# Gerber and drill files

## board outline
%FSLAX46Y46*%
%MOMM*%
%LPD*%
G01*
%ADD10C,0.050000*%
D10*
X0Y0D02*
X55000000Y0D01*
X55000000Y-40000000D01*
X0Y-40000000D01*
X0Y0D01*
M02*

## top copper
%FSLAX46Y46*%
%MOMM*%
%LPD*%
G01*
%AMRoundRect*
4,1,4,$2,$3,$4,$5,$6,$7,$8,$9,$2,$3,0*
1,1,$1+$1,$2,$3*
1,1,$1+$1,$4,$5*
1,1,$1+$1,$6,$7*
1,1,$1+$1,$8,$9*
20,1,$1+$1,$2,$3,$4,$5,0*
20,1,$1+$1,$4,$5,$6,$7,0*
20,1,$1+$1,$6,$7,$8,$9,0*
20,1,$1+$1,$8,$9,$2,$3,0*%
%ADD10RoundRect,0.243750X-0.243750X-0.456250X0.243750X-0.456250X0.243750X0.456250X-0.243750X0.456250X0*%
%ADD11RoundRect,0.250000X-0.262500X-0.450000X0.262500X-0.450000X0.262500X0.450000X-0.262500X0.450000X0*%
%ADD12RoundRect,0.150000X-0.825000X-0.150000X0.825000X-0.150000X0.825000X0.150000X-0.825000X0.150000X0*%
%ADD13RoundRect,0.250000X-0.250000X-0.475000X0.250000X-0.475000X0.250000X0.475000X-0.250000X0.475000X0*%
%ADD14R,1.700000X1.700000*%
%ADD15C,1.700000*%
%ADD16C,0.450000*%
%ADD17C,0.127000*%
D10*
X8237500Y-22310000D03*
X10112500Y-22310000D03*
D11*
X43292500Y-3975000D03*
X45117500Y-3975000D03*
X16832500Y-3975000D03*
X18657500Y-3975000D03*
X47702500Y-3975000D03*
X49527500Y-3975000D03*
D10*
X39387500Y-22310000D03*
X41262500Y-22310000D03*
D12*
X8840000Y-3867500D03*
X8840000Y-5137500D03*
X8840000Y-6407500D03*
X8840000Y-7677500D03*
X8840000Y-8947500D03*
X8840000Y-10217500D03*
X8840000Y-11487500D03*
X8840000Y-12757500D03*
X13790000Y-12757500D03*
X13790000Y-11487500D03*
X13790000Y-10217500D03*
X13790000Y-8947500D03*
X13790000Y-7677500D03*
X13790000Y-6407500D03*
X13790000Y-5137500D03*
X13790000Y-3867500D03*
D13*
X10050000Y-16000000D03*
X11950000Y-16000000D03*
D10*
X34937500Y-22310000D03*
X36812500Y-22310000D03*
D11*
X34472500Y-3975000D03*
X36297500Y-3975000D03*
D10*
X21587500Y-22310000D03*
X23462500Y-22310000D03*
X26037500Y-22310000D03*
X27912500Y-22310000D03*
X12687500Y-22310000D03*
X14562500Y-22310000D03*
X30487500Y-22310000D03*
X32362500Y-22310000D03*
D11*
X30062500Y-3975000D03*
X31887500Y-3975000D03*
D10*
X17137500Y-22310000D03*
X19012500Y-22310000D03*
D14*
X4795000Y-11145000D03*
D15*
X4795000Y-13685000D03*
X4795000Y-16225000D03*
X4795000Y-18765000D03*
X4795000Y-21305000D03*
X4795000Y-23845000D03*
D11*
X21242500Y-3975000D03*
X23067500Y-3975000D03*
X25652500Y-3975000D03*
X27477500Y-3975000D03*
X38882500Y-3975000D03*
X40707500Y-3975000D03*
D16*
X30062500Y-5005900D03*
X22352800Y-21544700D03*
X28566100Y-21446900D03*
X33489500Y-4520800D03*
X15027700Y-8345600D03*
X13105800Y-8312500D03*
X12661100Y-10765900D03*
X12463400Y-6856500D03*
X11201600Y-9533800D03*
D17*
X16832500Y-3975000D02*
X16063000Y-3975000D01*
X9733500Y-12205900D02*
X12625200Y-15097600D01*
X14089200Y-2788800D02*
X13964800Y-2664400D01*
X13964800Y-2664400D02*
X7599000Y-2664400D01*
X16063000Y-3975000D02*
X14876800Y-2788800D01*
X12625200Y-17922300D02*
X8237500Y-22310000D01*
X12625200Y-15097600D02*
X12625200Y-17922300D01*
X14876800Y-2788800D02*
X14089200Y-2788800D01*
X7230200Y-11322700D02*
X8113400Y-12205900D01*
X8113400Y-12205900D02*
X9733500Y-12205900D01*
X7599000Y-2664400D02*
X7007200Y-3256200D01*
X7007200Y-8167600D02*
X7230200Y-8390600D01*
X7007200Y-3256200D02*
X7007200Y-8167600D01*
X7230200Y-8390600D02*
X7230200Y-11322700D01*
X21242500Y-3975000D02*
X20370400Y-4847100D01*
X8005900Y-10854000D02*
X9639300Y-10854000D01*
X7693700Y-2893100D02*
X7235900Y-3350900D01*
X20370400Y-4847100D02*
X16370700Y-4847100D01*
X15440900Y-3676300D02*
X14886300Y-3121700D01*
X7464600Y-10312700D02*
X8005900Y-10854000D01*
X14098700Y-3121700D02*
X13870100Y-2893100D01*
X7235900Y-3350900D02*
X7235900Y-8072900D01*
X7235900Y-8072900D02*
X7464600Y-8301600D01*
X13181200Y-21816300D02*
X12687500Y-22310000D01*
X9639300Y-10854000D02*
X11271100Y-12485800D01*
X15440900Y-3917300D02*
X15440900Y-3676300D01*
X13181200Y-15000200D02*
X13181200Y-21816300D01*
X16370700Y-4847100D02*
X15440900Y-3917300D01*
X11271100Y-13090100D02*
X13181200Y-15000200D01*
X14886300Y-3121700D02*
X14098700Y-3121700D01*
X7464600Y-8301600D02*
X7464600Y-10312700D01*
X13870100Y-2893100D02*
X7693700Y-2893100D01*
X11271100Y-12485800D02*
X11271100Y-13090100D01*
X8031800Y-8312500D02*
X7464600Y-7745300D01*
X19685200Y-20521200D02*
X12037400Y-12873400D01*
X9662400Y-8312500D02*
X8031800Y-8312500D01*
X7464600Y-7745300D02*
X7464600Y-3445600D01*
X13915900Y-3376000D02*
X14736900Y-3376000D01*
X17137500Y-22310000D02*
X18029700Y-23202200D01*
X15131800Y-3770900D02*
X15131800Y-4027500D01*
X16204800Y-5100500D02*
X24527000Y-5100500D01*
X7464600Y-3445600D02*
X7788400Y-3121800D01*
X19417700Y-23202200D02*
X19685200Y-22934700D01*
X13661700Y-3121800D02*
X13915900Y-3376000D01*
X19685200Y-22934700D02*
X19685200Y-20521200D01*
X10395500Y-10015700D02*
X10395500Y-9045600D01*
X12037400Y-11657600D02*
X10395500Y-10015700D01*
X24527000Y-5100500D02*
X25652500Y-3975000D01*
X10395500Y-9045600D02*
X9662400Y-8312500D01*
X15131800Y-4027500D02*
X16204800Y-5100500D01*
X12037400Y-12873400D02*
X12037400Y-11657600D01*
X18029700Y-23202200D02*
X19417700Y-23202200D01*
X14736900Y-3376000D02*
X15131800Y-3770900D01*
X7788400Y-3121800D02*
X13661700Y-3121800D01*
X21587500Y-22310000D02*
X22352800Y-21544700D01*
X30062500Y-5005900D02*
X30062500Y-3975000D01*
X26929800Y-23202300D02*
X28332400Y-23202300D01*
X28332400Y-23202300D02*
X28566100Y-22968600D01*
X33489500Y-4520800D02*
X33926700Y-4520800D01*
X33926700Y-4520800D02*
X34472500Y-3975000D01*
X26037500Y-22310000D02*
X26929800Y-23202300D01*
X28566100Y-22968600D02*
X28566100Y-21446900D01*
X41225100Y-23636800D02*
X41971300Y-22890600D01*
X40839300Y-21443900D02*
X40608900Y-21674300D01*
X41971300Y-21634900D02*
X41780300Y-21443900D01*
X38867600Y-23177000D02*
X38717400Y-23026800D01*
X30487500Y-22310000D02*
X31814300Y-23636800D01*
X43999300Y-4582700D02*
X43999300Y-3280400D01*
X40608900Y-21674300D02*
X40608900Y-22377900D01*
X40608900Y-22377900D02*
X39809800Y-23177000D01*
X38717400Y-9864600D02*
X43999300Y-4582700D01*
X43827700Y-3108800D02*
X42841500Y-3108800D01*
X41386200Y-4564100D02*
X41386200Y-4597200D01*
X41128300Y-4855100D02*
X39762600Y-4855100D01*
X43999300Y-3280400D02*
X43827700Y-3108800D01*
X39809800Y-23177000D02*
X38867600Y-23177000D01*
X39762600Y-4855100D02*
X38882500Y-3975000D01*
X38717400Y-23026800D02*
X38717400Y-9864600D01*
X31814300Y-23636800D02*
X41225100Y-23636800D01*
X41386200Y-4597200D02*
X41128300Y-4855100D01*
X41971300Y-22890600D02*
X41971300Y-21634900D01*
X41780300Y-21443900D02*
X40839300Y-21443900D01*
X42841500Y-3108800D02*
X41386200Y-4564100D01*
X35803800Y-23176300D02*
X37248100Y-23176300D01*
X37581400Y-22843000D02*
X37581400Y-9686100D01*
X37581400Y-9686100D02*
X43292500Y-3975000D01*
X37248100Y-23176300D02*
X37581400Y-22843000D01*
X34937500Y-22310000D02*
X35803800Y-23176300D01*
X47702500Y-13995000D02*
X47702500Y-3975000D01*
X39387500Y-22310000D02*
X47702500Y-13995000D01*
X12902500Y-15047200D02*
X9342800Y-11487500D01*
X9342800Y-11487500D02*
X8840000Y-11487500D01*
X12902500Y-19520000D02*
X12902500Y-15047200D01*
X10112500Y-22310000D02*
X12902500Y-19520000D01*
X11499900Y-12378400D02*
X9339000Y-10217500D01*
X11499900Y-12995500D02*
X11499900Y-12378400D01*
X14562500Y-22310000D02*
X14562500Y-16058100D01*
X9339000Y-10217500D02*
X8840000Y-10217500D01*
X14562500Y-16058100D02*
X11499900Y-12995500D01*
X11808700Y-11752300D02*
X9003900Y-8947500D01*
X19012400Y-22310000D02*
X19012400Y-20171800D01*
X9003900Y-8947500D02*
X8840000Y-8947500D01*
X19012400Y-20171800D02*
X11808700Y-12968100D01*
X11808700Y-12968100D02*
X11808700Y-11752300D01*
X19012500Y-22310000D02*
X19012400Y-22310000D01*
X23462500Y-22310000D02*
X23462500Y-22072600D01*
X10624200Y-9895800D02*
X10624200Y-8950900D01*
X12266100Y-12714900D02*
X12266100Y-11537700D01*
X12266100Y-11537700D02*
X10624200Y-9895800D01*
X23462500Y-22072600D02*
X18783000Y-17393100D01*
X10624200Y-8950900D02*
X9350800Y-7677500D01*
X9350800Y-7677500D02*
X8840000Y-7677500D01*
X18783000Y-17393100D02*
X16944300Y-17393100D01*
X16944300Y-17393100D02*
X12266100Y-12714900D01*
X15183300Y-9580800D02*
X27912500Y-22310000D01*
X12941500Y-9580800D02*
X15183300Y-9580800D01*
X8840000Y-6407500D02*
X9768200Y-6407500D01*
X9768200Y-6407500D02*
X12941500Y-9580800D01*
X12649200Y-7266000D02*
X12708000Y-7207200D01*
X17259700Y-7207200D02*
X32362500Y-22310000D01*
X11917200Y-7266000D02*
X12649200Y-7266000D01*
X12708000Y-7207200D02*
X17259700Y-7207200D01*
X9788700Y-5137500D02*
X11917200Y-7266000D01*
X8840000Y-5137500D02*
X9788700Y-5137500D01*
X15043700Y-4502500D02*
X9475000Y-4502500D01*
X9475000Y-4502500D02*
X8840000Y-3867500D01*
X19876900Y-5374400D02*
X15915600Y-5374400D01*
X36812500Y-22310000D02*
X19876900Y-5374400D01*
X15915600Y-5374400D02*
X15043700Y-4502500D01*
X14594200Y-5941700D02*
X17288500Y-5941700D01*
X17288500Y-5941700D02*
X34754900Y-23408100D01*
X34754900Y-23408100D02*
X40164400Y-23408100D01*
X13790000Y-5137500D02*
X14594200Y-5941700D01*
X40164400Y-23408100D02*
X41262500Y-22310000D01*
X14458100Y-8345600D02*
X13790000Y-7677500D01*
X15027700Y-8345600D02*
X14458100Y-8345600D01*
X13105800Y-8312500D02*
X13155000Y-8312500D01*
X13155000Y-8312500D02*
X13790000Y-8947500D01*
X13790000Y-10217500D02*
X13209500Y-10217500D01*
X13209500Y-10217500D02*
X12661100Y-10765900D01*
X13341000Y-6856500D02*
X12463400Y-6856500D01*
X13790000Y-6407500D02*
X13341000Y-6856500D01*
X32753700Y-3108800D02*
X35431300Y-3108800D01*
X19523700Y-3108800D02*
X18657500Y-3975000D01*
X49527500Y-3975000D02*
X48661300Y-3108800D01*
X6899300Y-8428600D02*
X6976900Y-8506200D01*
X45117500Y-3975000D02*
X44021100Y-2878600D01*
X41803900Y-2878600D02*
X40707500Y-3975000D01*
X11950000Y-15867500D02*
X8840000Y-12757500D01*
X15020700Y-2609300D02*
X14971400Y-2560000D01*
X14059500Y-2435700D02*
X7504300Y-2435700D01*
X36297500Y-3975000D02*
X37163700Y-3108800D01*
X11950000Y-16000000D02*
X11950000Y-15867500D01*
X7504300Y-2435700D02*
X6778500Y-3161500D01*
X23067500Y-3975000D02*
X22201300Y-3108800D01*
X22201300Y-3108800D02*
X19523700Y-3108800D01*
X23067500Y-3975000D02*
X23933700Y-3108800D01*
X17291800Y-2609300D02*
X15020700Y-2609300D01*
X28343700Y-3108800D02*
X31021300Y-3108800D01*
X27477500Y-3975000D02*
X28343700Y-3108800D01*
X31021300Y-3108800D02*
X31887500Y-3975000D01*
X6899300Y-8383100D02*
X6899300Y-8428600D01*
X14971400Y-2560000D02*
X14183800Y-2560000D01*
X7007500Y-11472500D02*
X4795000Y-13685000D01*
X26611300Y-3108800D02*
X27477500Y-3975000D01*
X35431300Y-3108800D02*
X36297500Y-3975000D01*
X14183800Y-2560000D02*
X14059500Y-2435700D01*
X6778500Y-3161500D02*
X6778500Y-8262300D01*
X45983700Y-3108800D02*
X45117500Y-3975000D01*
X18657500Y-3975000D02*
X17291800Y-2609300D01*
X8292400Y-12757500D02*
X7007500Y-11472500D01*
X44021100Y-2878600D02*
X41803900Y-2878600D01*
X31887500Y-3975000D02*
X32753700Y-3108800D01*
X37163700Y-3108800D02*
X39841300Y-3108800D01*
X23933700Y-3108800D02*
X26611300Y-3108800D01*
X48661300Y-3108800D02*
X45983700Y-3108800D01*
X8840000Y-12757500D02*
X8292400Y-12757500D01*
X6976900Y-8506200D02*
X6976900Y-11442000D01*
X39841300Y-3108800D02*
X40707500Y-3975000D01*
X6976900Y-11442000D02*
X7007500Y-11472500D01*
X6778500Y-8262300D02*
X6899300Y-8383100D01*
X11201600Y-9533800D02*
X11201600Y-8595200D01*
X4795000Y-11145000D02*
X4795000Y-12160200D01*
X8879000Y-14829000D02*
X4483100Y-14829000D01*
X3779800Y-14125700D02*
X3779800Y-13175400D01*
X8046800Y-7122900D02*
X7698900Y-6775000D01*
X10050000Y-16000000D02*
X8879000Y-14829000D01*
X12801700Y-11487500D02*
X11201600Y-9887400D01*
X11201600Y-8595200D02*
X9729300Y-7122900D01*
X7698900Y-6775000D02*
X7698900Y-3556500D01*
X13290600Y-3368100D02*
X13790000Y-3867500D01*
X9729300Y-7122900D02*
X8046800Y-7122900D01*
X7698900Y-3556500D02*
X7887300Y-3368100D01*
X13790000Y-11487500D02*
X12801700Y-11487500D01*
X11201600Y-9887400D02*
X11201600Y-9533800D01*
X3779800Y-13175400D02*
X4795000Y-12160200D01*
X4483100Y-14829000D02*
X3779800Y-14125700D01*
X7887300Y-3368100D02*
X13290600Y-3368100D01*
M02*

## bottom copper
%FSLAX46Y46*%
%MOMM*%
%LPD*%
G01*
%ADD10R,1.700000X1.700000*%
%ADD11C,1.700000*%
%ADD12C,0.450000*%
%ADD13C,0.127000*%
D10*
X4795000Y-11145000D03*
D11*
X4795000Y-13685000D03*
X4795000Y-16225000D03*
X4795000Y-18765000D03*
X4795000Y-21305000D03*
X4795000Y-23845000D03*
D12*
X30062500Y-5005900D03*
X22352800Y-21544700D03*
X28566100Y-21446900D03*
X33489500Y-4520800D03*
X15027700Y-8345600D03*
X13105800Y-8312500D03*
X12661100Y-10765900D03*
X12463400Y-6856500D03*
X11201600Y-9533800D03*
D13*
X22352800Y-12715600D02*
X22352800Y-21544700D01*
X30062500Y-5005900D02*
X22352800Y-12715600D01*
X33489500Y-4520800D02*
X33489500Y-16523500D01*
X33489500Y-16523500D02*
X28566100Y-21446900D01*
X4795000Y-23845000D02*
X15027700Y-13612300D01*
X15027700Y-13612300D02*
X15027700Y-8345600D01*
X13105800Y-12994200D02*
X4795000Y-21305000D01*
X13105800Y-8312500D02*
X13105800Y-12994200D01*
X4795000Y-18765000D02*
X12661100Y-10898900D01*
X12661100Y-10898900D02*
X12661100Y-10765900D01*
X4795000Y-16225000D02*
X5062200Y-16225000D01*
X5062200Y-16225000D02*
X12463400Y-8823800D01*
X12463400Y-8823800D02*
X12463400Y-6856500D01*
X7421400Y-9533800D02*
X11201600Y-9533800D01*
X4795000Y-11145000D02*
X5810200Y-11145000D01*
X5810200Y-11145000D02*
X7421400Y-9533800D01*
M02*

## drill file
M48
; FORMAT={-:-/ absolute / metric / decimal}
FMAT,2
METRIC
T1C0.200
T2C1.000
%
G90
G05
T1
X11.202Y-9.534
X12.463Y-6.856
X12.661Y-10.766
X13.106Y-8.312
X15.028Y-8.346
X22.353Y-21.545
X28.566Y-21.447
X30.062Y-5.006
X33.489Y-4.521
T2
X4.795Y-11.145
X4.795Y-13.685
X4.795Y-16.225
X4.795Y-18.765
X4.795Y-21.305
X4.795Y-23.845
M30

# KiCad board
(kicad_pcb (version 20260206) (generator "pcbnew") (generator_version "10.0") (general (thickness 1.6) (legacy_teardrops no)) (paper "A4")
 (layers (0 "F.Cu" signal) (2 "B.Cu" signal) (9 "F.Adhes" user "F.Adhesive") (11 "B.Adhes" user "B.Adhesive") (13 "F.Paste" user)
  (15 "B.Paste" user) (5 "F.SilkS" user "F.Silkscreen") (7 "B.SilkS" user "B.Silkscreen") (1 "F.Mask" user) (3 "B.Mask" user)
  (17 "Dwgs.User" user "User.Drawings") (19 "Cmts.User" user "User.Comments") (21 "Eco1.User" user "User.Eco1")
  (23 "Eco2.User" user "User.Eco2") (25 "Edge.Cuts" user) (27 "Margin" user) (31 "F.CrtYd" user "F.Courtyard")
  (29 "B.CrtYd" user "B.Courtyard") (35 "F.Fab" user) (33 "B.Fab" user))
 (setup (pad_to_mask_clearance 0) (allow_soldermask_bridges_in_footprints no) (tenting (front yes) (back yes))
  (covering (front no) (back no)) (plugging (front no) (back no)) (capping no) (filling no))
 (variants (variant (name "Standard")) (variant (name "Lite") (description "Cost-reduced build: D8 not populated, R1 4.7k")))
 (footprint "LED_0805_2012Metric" (layer "F.Cu") (at 9.175 22.31)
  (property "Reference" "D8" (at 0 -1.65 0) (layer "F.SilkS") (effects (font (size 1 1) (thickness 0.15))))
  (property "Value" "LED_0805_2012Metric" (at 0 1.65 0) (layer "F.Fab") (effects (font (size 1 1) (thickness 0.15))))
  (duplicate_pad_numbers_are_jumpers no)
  (pad "1" smd roundrect (at -0.9375 0) (size 0.975 1.4) (layers "F.Cu" "F.Mask" "F.Paste") (roundrect_rratio 0.25) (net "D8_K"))
  (pad "2" smd roundrect (at 0.9375 0) (size 0.975 1.4) (layers "F.Cu" "F.Mask" "F.Paste") (roundrect_rratio 0.25) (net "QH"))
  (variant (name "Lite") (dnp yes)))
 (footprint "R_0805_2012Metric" (layer "F.Cu") (at 44.205 3.975)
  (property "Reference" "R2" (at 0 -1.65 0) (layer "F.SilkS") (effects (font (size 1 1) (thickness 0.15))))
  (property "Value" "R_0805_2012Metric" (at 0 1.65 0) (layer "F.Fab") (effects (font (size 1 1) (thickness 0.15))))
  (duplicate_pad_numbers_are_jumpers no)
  (pad "1" smd roundrect (at -0.9125 0) (size 1.025 1.4) (layers "F.Cu" "F.Mask" "F.Paste") (roundrect_rratio 0.243902) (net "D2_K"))
  (pad "2" smd roundrect (at 0.9125 0) (size 1.025 1.4) (layers "F.Cu" "F.Mask" "F.Paste") (roundrect_rratio 0.243902) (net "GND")))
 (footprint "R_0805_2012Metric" (layer "F.Cu") (at 17.745 3.975)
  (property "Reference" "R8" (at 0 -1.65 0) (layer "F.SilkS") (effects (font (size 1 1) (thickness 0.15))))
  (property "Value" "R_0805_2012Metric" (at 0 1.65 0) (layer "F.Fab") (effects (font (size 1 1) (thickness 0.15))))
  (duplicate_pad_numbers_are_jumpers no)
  (pad "1" smd roundrect (at -0.9125 0) (size 1.025 1.4) (layers "F.Cu" "F.Mask" "F.Paste") (roundrect_rratio 0.243902) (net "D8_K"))
  (pad "2" smd roundrect (at 0.9125 0) (size 1.025 1.4) (layers "F.Cu" "F.Mask" "F.Paste") (roundrect_rratio 0.243902) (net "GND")))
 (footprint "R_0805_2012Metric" (layer "F.Cu") (at 48.615 3.975)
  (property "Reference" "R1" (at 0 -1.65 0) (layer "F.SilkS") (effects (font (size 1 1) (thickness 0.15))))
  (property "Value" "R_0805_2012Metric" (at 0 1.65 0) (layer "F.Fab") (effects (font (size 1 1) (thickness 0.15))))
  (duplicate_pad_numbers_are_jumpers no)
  (pad "1" smd roundrect (at -0.9125 0) (size 1.025 1.4) (layers "F.Cu" "F.Mask" "F.Paste") (roundrect_rratio 0.243902) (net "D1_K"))
  (pad "2" smd roundrect (at 0.9125 0) (size 1.025 1.4) (layers "F.Cu" "F.Mask" "F.Paste") (roundrect_rratio 0.243902) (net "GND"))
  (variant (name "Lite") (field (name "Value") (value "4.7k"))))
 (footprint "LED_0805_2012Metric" (layer "F.Cu") (at 40.325 22.31)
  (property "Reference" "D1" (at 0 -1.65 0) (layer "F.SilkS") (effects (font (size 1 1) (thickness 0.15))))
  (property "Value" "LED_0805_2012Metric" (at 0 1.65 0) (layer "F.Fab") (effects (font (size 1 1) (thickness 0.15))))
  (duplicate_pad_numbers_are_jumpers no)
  (pad "1" smd roundrect (at -0.9375 0) (size 0.975 1.4) (layers "F.Cu" "F.Mask" "F.Paste") (roundrect_rratio 0.25) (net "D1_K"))
  (pad "2" smd roundrect (at 0.9375 0) (size 0.975 1.4) (layers "F.Cu" "F.Mask" "F.Paste") (roundrect_rratio 0.25) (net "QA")))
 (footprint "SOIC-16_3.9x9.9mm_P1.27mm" (layer "F.Cu") (at 11.315 8.3125)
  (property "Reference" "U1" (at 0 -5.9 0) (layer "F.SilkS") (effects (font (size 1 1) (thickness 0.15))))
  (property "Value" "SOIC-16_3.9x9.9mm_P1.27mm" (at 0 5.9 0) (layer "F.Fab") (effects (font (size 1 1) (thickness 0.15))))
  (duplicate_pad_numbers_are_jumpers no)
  (pad "1" smd roundrect (at -2.475 -4.445) (size 1.95 0.6) (layers "F.Cu" "F.Mask" "F.Paste") (roundrect_rratio 0.25) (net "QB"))
  (pad "2" smd roundrect (at -2.475 -3.175) (size 1.95 0.6) (layers "F.Cu" "F.Mask" "F.Paste") (roundrect_rratio 0.25) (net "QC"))
  (pad "3" smd roundrect (at -2.475 -1.905) (size 1.95 0.6) (layers "F.Cu" "F.Mask" "F.Paste") (roundrect_rratio 0.25) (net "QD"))
  (pad "4" smd roundrect (at -2.475 -0.635) (size 1.95 0.6) (layers "F.Cu" "F.Mask" "F.Paste") (roundrect_rratio 0.25) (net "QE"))
  (pad "5" smd roundrect (at -2.475 0.635) (size 1.95 0.6) (layers "F.Cu" "F.Mask" "F.Paste") (roundrect_rratio 0.25) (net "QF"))
  (pad "6" smd roundrect (at -2.475 1.905) (size 1.95 0.6) (layers "F.Cu" "F.Mask" "F.Paste") (roundrect_rratio 0.25) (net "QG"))
  (pad "7" smd roundrect (at -2.475 3.175) (size 1.95 0.6) (layers "F.Cu" "F.Mask" "F.Paste") (roundrect_rratio 0.25) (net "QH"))
  (pad "8" smd roundrect (at -2.475 4.445) (size 1.95 0.6) (layers "F.Cu" "F.Mask" "F.Paste") (roundrect_rratio 0.25) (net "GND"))
  (pad "9" smd roundrect (at 2.475 4.445) (size 1.95 0.6) (layers "F.Cu" "F.Mask" "F.Paste") (roundrect_rratio 0.25) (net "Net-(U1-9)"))
  (pad "10" smd roundrect (at 2.475 3.175) (size 1.95 0.6) (layers "F.Cu" "F.Mask" "F.Paste") (roundrect_rratio 0.25) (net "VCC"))
  (pad "11" smd roundrect (at 2.475 1.905) (size 1.95 0.6) (layers "F.Cu" "F.Mask" "F.Paste") (roundrect_rratio 0.25) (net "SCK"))
  (pad "12" smd roundrect (at 2.475 0.635) (size 1.95 0.6) (layers "F.Cu" "F.Mask" "F.Paste") (roundrect_rratio 0.25) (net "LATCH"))
  (pad "13" smd roundrect (at 2.475 -0.635) (size 1.95 0.6) (layers "F.Cu" "F.Mask" "F.Paste") (roundrect_rratio 0.25) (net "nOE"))
  (pad "14" smd roundrect (at 2.475 -1.905) (size 1.95 0.6) (layers "F.Cu" "F.Mask" "F.Paste") (roundrect_rratio 0.25) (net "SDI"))
  (pad "15" smd roundrect (at 2.475 -3.175) (size 1.95 0.6) (layers "F.Cu" "F.Mask" "F.Paste") (roundrect_rratio 0.25) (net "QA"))
  (pad "16" smd roundrect (at 2.475 -4.445) (size 1.95 0.6) (layers "F.Cu" "F.Mask" "F.Paste") (roundrect_rratio 0.25) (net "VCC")))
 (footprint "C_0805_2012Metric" (layer "F.Cu") (at 11 16)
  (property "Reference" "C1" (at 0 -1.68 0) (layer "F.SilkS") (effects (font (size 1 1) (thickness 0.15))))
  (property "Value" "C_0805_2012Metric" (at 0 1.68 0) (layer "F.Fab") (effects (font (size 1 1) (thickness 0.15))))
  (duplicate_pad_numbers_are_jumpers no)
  (pad "1" smd roundrect (at -0.95 0) (size 1 1.45) (layers "F.Cu" "F.Mask" "F.Paste") (roundrect_rratio 0.25) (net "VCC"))
  (pad "2" smd roundrect (at 0.95 0) (size 1 1.45) (layers "F.Cu" "F.Mask" "F.Paste") (roundrect_rratio 0.25) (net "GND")))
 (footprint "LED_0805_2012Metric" (layer "F.Cu") (at 35.875 22.31)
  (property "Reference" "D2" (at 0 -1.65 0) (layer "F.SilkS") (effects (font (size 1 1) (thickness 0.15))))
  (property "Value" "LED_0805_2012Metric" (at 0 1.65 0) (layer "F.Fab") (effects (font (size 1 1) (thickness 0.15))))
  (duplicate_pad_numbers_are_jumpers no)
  (pad "1" smd roundrect (at -0.9375 0) (size 0.975 1.4) (layers "F.Cu" "F.Mask" "F.Paste") (roundrect_rratio 0.25) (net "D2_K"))
  (pad "2" smd roundrect (at 0.9375 0) (size 0.975 1.4) (layers "F.Cu" "F.Mask" "F.Paste") (roundrect_rratio 0.25) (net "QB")))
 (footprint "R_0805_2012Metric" (layer "F.Cu") (at 35.385 3.975)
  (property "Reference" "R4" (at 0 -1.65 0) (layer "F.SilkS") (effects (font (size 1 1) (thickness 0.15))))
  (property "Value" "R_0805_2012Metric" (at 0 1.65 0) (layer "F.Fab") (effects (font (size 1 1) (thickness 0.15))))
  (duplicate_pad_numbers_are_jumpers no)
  (pad "1" smd roundrect (at -0.9125 0) (size 1.025 1.4) (layers "F.Cu" "F.Mask" "F.Paste") (roundrect_rratio 0.243902) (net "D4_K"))
  (pad "2" smd roundrect (at 0.9125 0) (size 1.025 1.4) (layers "F.Cu" "F.Mask" "F.Paste") (roundrect_rratio 0.243902) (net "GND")))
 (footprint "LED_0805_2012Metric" (layer "F.Cu") (at 22.525 22.31)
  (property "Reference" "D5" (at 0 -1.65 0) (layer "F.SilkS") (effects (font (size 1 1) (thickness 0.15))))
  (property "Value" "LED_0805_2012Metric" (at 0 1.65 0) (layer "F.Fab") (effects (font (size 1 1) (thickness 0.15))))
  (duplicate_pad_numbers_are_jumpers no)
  (pad "1" smd roundrect (at -0.9375 0) (size 0.975 1.4) (layers "F.Cu" "F.Mask" "F.Paste") (roundrect_rratio 0.25) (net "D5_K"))
  (pad "2" smd roundrect (at 0.9375 0) (size 0.975 1.4) (layers "F.Cu" "F.Mask" "F.Paste") (roundrect_rratio 0.25) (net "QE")))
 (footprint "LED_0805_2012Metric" (layer "F.Cu") (at 26.975 22.31)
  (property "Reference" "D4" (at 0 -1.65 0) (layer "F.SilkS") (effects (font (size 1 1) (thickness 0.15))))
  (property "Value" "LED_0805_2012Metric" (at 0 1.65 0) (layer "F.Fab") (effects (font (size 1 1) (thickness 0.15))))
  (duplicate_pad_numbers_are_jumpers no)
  (pad "1" smd roundrect (at -0.9375 0) (size 0.975 1.4) (layers "F.Cu" "F.Mask" "F.Paste") (roundrect_rratio 0.25) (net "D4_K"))
  (pad "2" smd roundrect (at 0.9375 0) (size 0.975 1.4) (layers "F.Cu" "F.Mask" "F.Paste") (roundrect_rratio 0.25) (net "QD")))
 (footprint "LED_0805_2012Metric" (layer "F.Cu") (at 13.625 22.31)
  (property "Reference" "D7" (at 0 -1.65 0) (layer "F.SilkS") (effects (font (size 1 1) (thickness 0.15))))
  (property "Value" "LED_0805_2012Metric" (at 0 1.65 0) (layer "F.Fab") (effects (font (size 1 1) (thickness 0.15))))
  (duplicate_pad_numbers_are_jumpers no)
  (pad "1" smd roundrect (at -0.9375 0) (size 0.975 1.4) (layers "F.Cu" "F.Mask" "F.Paste") (roundrect_rratio 0.25) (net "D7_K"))
  (pad "2" smd roundrect (at 0.9375 0) (size 0.975 1.4) (layers "F.Cu" "F.Mask" "F.Paste") (roundrect_rratio 0.25) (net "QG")))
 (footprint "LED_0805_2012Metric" (layer "F.Cu") (at 31.425 22.31)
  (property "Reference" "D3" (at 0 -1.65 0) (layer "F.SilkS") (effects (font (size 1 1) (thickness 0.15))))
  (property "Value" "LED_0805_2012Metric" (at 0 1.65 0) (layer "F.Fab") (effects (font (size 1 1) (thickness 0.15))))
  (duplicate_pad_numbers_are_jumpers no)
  (pad "1" smd roundrect (at -0.9375 0) (size 0.975 1.4) (layers "F.Cu" "F.Mask" "F.Paste") (roundrect_rratio 0.25) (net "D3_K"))
  (pad "2" smd roundrect (at 0.9375 0) (size 0.975 1.4) (layers "F.Cu" "F.Mask" "F.Paste") (roundrect_rratio 0.25) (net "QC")))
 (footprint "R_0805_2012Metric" (layer "F.Cu") (at 30.975 3.975)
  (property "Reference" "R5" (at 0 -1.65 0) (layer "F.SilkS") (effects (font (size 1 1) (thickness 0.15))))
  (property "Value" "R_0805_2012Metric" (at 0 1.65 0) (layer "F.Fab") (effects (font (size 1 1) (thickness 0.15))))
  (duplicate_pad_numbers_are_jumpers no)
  (pad "1" smd roundrect (at -0.9125 0) (size 1.025 1.4) (layers "F.Cu" "F.Mask" "F.Paste") (roundrect_rratio 0.243902) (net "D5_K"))
  (pad "2" smd roundrect (at 0.9125 0) (size 1.025 1.4) (layers "F.Cu" "F.Mask" "F.Paste") (roundrect_rratio 0.243902) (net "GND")))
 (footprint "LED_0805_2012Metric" (layer "F.Cu") (at 18.075 22.31)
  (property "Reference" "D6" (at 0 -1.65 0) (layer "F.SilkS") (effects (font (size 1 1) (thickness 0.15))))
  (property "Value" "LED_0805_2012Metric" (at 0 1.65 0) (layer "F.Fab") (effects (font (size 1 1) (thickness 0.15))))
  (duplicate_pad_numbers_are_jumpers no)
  (pad "1" smd roundrect (at -0.9375 0) (size 0.975 1.4) (layers "F.Cu" "F.Mask" "F.Paste") (roundrect_rratio 0.25) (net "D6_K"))
  (pad "2" smd roundrect (at 0.9375 0) (size 0.975 1.4) (layers "F.Cu" "F.Mask" "F.Paste") (roundrect_rratio 0.25) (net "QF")))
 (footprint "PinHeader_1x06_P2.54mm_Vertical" (layer "F.Cu") (at 4.795 11.145)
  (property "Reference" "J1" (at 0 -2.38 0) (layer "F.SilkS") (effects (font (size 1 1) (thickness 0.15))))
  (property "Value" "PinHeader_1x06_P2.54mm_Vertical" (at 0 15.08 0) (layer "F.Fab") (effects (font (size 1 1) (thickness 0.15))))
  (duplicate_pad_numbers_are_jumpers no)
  (pad "1" thru_hole rect (at 0 0) (size 1.7 1.7) (drill 1) (layers "*.Cu" "*.Mask") (remove_unused_layers no) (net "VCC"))
  (pad "2" thru_hole circle (at 0 2.54) (size 1.7 1.7) (drill 1) (layers "*.Cu" "*.Mask") (remove_unused_layers no) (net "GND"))
  (pad "3" thru_hole circle (at 0 5.08) (size 1.7 1.7) (drill 1) (layers "*.Cu" "*.Mask") (remove_unused_layers no) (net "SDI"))
  (pad "4" thru_hole circle (at 0 7.62) (size 1.7 1.7) (drill 1) (layers "*.Cu" "*.Mask") (remove_unused_layers no) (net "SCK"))
  (pad "5" thru_hole circle (at 0 10.16) (size 1.7 1.7) (drill 1) (layers "*.Cu" "*.Mask") (remove_unused_layers no) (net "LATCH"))
  (pad "6" thru_hole circle (at 0 12.7) (size 1.7 1.7) (drill 1) (layers "*.Cu" "*.Mask") (remove_unused_layers no) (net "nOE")))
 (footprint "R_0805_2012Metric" (layer "F.Cu") (at 22.155 3.975)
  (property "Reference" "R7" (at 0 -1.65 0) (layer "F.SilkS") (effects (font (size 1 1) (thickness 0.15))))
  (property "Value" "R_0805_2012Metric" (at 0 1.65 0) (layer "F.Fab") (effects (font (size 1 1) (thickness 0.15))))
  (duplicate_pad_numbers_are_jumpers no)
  (pad "1" smd roundrect (at -0.9125 0) (size 1.025 1.4) (layers "F.Cu" "F.Mask" "F.Paste") (roundrect_rratio 0.243902) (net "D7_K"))
  (pad "2" smd roundrect (at 0.9125 0) (size 1.025 1.4) (layers "F.Cu" "F.Mask" "F.Paste") (roundrect_rratio 0.243902) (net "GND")))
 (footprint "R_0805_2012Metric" (layer "F.Cu") (at 26.565 3.975)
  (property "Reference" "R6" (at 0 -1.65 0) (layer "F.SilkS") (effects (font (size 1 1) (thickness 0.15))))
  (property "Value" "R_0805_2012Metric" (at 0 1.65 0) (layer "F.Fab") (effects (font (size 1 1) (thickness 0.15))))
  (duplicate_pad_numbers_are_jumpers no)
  (pad "1" smd roundrect (at -0.9125 0) (size 1.025 1.4) (layers "F.Cu" "F.Mask" "F.Paste") (roundrect_rratio 0.243902) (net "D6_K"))
  (pad "2" smd roundrect (at 0.9125 0) (size 1.025 1.4) (layers "F.Cu" "F.Mask" "F.Paste") (roundrect_rratio 0.243902) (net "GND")))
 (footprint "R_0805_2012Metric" (layer "F.Cu") (at 39.795 3.975)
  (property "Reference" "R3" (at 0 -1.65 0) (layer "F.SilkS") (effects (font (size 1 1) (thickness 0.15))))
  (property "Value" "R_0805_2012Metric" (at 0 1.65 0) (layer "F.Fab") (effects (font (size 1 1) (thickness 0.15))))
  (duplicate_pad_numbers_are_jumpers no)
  (pad "1" smd roundrect (at -0.9125 0) (size 1.025 1.4) (layers "F.Cu" "F.Mask" "F.Paste") (roundrect_rratio 0.243902) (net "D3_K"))
  (pad "2" smd roundrect (at 0.9125 0) (size 1.025 1.4) (layers "F.Cu" "F.Mask" "F.Paste") (roundrect_rratio 0.243902) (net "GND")))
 (gr_rect (start 0 0) (end 55 40) (stroke (width 0.05) (type default)) (fill no) (layer "Edge.Cuts"))
 (segment (start 16.8325 3.975) (end 16.063 3.975) (width 0.127) (layer "F.Cu") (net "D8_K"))
 (segment (start 9.7335 12.2059) (end 12.6252 15.0976) (width 0.127) (layer "F.Cu") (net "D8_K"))
 (segment (start 14.0892 2.7888) (end 13.9648 2.6644) (width 0.127) (layer "F.Cu") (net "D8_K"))
 (segment (start 13.9648 2.6644) (end 7.599 2.6644) (width 0.127) (layer "F.Cu") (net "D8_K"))
 (segment (start 16.063 3.975) (end 14.8768 2.7888) (width 0.127) (layer "F.Cu") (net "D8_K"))
 (segment (start 12.6252 17.9223) (end 8.2375 22.31) (width 0.127) (layer "F.Cu") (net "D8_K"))
 (segment (start 12.6252 15.0976) (end 12.6252 17.9223) (width 0.127) (layer "F.Cu") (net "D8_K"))
 (segment (start 14.8768 2.7888) (end 14.0892 2.7888) (width 0.127) (layer "F.Cu") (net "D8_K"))
 (segment (start 7.2302 11.3227) (end 8.1134 12.2059) (width 0.127) (layer "F.Cu") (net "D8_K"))
 (segment (start 8.1134 12.2059) (end 9.7335 12.2059) (width 0.127) (layer "F.Cu") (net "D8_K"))
 (segment (start 7.599 2.6644) (end 7.0072 3.2562) (width 0.127) (layer "F.Cu") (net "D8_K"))
 (segment (start 7.0072 8.1676) (end 7.2302 8.3906) (width 0.127) (layer "F.Cu") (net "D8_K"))
 (segment (start 7.0072 3.2562) (end 7.0072 8.1676) (width 0.127) (layer "F.Cu") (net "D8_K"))
 (segment (start 7.2302 8.3906) (end 7.2302 11.3227) (width 0.127) (layer "F.Cu") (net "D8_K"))
 (segment (start 21.2425 3.975) (end 20.3704 4.8471) (width 0.127) (layer "F.Cu") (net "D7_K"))
 (segment (start 8.0059 10.854) (end 9.6393 10.854) (width 0.127) (layer "F.Cu") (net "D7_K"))
 (segment (start 7.6937 2.8931) (end 7.2359 3.3509) (width 0.127) (layer "F.Cu") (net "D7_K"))
 (segment (start 20.3704 4.8471) (end 16.3707 4.8471) (width 0.127) (layer "F.Cu") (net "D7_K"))
 (segment (start 15.4409 3.6763) (end 14.8863 3.1217) (width 0.127) (layer "F.Cu") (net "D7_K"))
 (segment (start 7.4646 10.3127) (end 8.0059 10.854) (width 0.127) (layer "F.Cu") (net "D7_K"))
 (segment (start 14.0987 3.1217) (end 13.8701 2.8931) (width 0.127) (layer "F.Cu") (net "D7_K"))
 (segment (start 7.2359 3.3509) (end 7.2359 8.0729) (width 0.127) (layer "F.Cu") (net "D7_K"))
 (segment (start 7.2359 8.0729) (end 7.4646 8.3016) (width 0.127) (layer "F.Cu") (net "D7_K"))
 (segment (start 13.1812 21.8163) (end 12.6875 22.31) (width 0.127) (layer "F.Cu") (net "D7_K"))
 (segment (start 9.6393 10.854) (end 11.2711 12.4858) (width 0.127) (layer "F.Cu") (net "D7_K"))
 (segment (start 15.4409 3.9173) (end 15.4409 3.6763) (width 0.127) (layer "F.Cu") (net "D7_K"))
 (segment (start 13.1812 15.0002) (end 13.1812 21.8163) (width 0.127) (layer "F.Cu") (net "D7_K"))
 (segment (start 16.3707 4.8471) (end 15.4409 3.9173) (width 0.127) (layer "F.Cu") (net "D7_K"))
 (segment (start 11.2711 13.0901) (end 13.1812 15.0002) (width 0.127) (layer "F.Cu") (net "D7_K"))
 (segment (start 14.8863 3.1217) (end 14.0987 3.1217) (width 0.127) (layer "F.Cu") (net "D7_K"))
 (segment (start 7.4646 8.3016) (end 7.4646 10.3127) (width 0.127) (layer "F.Cu") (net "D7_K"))
 (segment (start 13.8701 2.8931) (end 7.6937 2.8931) (width 0.127) (layer "F.Cu") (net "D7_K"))
 (segment (start 11.2711 12.4858) (end 11.2711 13.0901) (width 0.127) (layer "F.Cu") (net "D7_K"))
 (segment (start 8.0318 8.3125) (end 7.4646 7.7453) (width 0.127) (layer "F.Cu") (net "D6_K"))
 (segment (start 19.6852 20.5212) (end 12.0374 12.8734) (width 0.127) (layer "F.Cu") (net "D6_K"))
 (segment (start 9.6624 8.3125) (end 8.0318 8.3125) (width 0.127) (layer "F.Cu") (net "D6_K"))
 (segment (start 7.4646 7.7453) (end 7.4646 3.4456) (width 0.127) (layer "F.Cu") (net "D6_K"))
 (segment (start 13.9159 3.376) (end 14.7369 3.376) (width 0.127) (layer "F.Cu") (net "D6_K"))
 (segment (start 17.1375 22.31) (end 18.0297 23.2022) (width 0.127) (layer "F.Cu") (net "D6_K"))
 (segment (start 15.1318 3.7709) (end 15.1318 4.0275) (width 0.127) (layer "F.Cu") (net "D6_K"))
 (segment (start 16.2048 5.1005) (end 24.527 5.1005) (width 0.127) (layer "F.Cu") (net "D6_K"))
 (segment (start 7.4646 3.4456) (end 7.7884 3.1218) (width 0.127) (layer "F.Cu") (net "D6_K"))
 (segment (start 19.4177 23.2022) (end 19.6852 22.9347) (width 0.127) (layer "F.Cu") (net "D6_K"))
 (segment (start 13.6617 3.1218) (end 13.9159 3.376) (width 0.127) (layer "F.Cu") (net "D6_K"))
 (segment (start 19.6852 22.9347) (end 19.6852 20.5212) (width 0.127) (layer "F.Cu") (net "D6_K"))
 (segment (start 10.3955 10.0157) (end 10.3955 9.0456) (width 0.127) (layer "F.Cu") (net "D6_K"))
 (segment (start 12.0374 11.6576) (end 10.3955 10.0157) (width 0.127) (layer "F.Cu") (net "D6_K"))
 (segment (start 24.527 5.1005) (end 25.6525 3.975) (width 0.127) (layer "F.Cu") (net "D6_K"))
 (segment (start 10.3955 9.0456) (end 9.6624 8.3125) (width 0.127) (layer "F.Cu") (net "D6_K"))
 (segment (start 15.1318 4.0275) (end 16.2048 5.1005) (width 0.127) (layer "F.Cu") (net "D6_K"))
 (segment (start 12.0374 12.8734) (end 12.0374 11.6576) (width 0.127) (layer "F.Cu") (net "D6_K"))
 (segment (start 18.0297 23.2022) (end 19.4177 23.2022) (width 0.127) (layer "F.Cu") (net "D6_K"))
 (segment (start 14.7369 3.376) (end 15.1318 3.7709) (width 0.127) (layer "F.Cu") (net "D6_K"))
 (segment (start 7.7884 3.1218) (end 13.6617 3.1218) (width 0.127) (layer "F.Cu") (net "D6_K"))
 (segment (start 21.5875 22.31) (end 22.3528 21.5447) (width 0.127) (layer "F.Cu") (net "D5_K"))
 (segment (start 30.0625 5.0059) (end 30.0625 3.975) (width 0.127) (layer "F.Cu") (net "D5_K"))
 (via (at 30.0625 5.0059) (size 0.45) (drill 0.2) (layers "F.Cu" "B.Cu") (capping no) (covering (front no) (back no))
  (plugging (front no) (back no)) (filling no) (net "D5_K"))
 (via (at 22.3528 21.5447) (size 0.45) (drill 0.2) (layers "F.Cu" "B.Cu") (capping no) (covering (front no) (back no))
  (plugging (front no) (back no)) (filling no) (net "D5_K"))
 (segment (start 22.3528 12.7156) (end 22.3528 21.5447) (width 0.127) (layer "B.Cu") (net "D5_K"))
 (segment (start 30.0625 5.0059) (end 22.3528 12.7156) (width 0.127) (layer "B.Cu") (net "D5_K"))
 (segment (start 26.9298 23.2023) (end 28.3324 23.2023) (width 0.127) (layer "F.Cu") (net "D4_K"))
 (segment (start 28.3324 23.2023) (end 28.5661 22.9686) (width 0.127) (layer "F.Cu") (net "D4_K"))
 (segment (start 33.4895 4.5208) (end 33.9267 4.5208) (width 0.127) (layer "F.Cu") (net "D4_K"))
 (segment (start 33.9267 4.5208) (end 34.4725 3.975) (width 0.127) (layer "F.Cu") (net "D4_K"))
 (segment (start 26.0375 22.31) (end 26.9298 23.2023) (width 0.127) (layer "F.Cu") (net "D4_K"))
 (segment (start 28.5661 22.9686) (end 28.5661 21.4469) (width 0.127) (layer "F.Cu") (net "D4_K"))
 (via (at 28.5661 21.4469) (size 0.45) (drill 0.2) (layers "F.Cu" "B.Cu") (capping no) (covering (front no) (back no))
  (plugging (front no) (back no)) (filling no) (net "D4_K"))
 (via (at 33.4895 4.5208) (size 0.45) (drill 0.2) (layers "F.Cu" "B.Cu") (capping no) (covering (front no) (back no))
  (plugging (front no) (back no)) (filling no) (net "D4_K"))
 (segment (start 33.4895 4.5208) (end 33.4895 16.5235) (width 0.127) (layer "B.Cu") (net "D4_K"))
 (segment (start 33.4895 16.5235) (end 28.5661 21.4469) (width 0.127) (layer "B.Cu") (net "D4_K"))
 (segment (start 41.2251 23.6368) (end 41.9713 22.8906) (width 0.127) (layer "F.Cu") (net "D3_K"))
 (segment (start 40.8393 21.4439) (end 40.6089 21.6743) (width 0.127) (layer "F.Cu") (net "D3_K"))
 (segment (start 41.9713 21.6349) (end 41.7803 21.4439) (width 0.127) (layer "F.Cu") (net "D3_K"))
 (segment (start 38.8676 23.177) (end 38.7174 23.0268) (width 0.127) (layer "F.Cu") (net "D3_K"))
 (segment (start 30.4875 22.31) (end 31.8143 23.6368) (width 0.127) (layer "F.Cu") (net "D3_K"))
 (segment (start 43.9993 4.5827) (end 43.9993 3.2804) (width 0.127) (layer "F.Cu") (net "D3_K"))
 (segment (start 40.6089 21.6743) (end 40.6089 22.3779) (width 0.127) (layer "F.Cu") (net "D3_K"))
 (segment (start 40.6089 22.3779) (end 39.8098 23.177) (width 0.127) (layer "F.Cu") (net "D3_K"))
 (segment (start 38.7174 9.8646) (end 43.9993 4.5827) (width 0.127) (layer "F.Cu") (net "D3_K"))
 (segment (start 43.8277 3.1088) (end 42.8415 3.1088) (width 0.127) (layer "F.Cu") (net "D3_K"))
 (segment (start 41.3862 4.5641) (end 41.3862 4.5972) (width 0.127) (layer "F.Cu") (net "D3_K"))
 (segment (start 41.1283 4.8551) (end 39.7626 4.8551) (width 0.127) (layer "F.Cu") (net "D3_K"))
 (segment (start 43.9993 3.2804) (end 43.8277 3.1088) (width 0.127) (layer "F.Cu") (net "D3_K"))
 (segment (start 39.8098 23.177) (end 38.8676 23.177) (width 0.127) (layer "F.Cu") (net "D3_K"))
 (segment (start 39.7626 4.8551) (end 38.8825 3.975) (width 0.127) (layer "F.Cu") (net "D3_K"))
 (segment (start 38.7174 23.0268) (end 38.7174 9.8646) (width 0.127) (layer "F.Cu") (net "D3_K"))
 (segment (start 31.8143 23.6368) (end 41.2251 23.6368) (width 0.127) (layer "F.Cu") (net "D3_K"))
 (segment (start 41.3862 4.5972) (end 41.1283 4.8551) (width 0.127) (layer "F.Cu") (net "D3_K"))
 (segment (start 41.9713 22.8906) (end 41.9713 21.6349) (width 0.127) (layer "F.Cu") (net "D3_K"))
 (segment (start 41.7803 21.4439) (end 40.8393 21.4439) (width 0.127) (layer "F.Cu") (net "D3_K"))
 (segment (start 42.8415 3.1088) (end 41.3862 4.5641) (width 0.127) (layer "F.Cu") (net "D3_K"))
 (segment (start 35.8038 23.1763) (end 37.2481 23.1763) (width 0.127) (layer "F.Cu") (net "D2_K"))
 (segment (start 37.5814 22.843) (end 37.5814 9.6861) (width 0.127) (layer "F.Cu") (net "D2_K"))
 (segment (start 37.5814 9.6861) (end 43.2925 3.975) (width 0.127) (layer "F.Cu") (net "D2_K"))
 (segment (start 37.2481 23.1763) (end 37.5814 22.843) (width 0.127) (layer "F.Cu") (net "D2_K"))
 (segment (start 34.9375 22.31) (end 35.8038 23.1763) (width 0.127) (layer "F.Cu") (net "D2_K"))
 (segment (start 47.7025 13.995) (end 47.7025 3.975) (width 0.127) (layer "F.Cu") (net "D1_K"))
 (segment (start 39.3875 22.31) (end 47.7025 13.995) (width 0.127) (layer "F.Cu") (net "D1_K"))
 (segment (start 12.9025 15.0472) (end 9.3428 11.4875) (width 0.127) (layer "F.Cu") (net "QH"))
 (segment (start 9.3428 11.4875) (end 8.84 11.4875) (width 0.127) (layer "F.Cu") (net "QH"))
 (segment (start 12.9025 19.52) (end 12.9025 15.0472) (width 0.127) (layer "F.Cu") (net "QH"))
 (segment (start 10.1125 22.31) (end 12.9025 19.52) (width 0.127) (layer "F.Cu") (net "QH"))
 (segment (start 11.4999 12.3784) (end 9.339 10.2175) (width 0.127) (layer "F.Cu") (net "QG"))
 (segment (start 11.4999 12.9955) (end 11.4999 12.3784) (width 0.127) (layer "F.Cu") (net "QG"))
 (segment (start 14.5625 22.31) (end 14.5625 16.0581) (width 0.127) (layer "F.Cu") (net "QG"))
 (segment (start 9.339 10.2175) (end 8.84 10.2175) (width 0.127) (layer "F.Cu") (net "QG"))
 (segment (start 14.5625 16.0581) (end 11.4999 12.9955) (width 0.127) (layer "F.Cu") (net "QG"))
 (segment (start 11.8087 11.7523) (end 9.0039 8.9475) (width 0.127) (layer "F.Cu") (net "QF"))
 (segment (start 19.0124 22.31) (end 19.0124 20.1718) (width 0.127) (layer "F.Cu") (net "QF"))
 (segment (start 9.0039 8.9475) (end 8.84 8.9475) (width 0.127) (layer "F.Cu") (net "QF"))
 (segment (start 19.0124 20.1718) (end 11.8087 12.9681) (width 0.127) (layer "F.Cu") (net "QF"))
 (segment (start 11.8087 12.9681) (end 11.8087 11.7523) (width 0.127) (layer "F.Cu") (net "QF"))
 (segment (start 19.0125 22.31) (end 19.0124 22.31) (width 0.127) (layer "F.Cu") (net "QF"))
 (segment (start 23.4625 22.31) (end 23.4625 22.0726) (width 0.127) (layer "F.Cu") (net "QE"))
 (segment (start 10.6242 9.8958) (end 10.6242 8.9509) (width 0.127) (layer "F.Cu") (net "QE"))
 (segment (start 12.2661 12.7149) (end 12.2661 11.5377) (width 0.127) (layer "F.Cu") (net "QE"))
 (segment (start 12.2661 11.5377) (end 10.6242 9.8958) (width 0.127) (layer "F.Cu") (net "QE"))
 (segment (start 23.4625 22.0726) (end 18.783 17.3931) (width 0.127) (layer "F.Cu") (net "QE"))
 (segment (start 10.6242 8.9509) (end 9.3508 7.6775) (width 0.127) (layer "F.Cu") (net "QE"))
 (segment (start 9.3508 7.6775) (end 8.84 7.6775) (width 0.127) (layer "F.Cu") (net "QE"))
 (segment (start 18.783 17.3931) (end 16.9443 17.3931) (width 0.127) (layer "F.Cu") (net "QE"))
 (segment (start 16.9443 17.3931) (end 12.2661 12.7149) (width 0.127) (layer "F.Cu") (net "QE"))
 (segment (start 15.1833 9.5808) (end 27.9125 22.31) (width 0.127) (layer "F.Cu") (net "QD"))
 (segment (start 12.9415 9.5808) (end 15.1833 9.5808) (width 0.127) (layer "F.Cu") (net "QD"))
 (segment (start 8.84 6.4075) (end 9.7682 6.4075) (width 0.127) (layer "F.Cu") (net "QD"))
 (segment (start 9.7682 6.4075) (end 12.9415 9.5808) (width 0.127) (layer "F.Cu") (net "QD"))
 (segment (start 12.6492 7.266) (end 12.708 7.2072) (width 0.127) (layer "F.Cu") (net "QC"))
 (segment (start 17.2597 7.2072) (end 32.3625 22.31) (width 0.127) (layer "F.Cu") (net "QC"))
 (segment (start 11.9172 7.266) (end 12.6492 7.266) (width 0.127) (layer "F.Cu") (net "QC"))
 (segment (start 12.708 7.2072) (end 17.2597 7.2072) (width 0.127) (layer "F.Cu") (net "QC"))
 (segment (start 9.7887 5.1375) (end 11.9172 7.266) (width 0.127) (layer "F.Cu") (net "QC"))
 (segment (start 8.84 5.1375) (end 9.7887 5.1375) (width 0.127) (layer "F.Cu") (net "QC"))
 (segment (start 15.0437 4.5025) (end 9.475 4.5025) (width 0.127) (layer "F.Cu") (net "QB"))
 (segment (start 9.475 4.5025) (end 8.84 3.8675) (width 0.127) (layer "F.Cu") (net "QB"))
 (segment (start 19.8769 5.3744) (end 15.9156 5.3744) (width 0.127) (layer "F.Cu") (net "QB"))
 (segment (start 36.8125 22.31) (end 19.8769 5.3744) (width 0.127) (layer "F.Cu") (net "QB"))
 (segment (start 15.9156 5.3744) (end 15.0437 4.5025) (width 0.127) (layer "F.Cu") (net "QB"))
 (segment (start 14.5942 5.9417) (end 17.2885 5.9417) (width 0.127) (layer "F.Cu") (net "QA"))
 (segment (start 17.2885 5.9417) (end 34.7549 23.4081) (width 0.127) (layer "F.Cu") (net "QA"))
 (segment (start 34.7549 23.4081) (end 40.1644 23.4081) (width 0.127) (layer "F.Cu") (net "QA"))
 (segment (start 13.79 5.1375) (end 14.5942 5.9417) (width 0.127) (layer "F.Cu") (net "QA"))
 (segment (start 40.1644 23.4081) (end 41.2625 22.31) (width 0.127) (layer "F.Cu") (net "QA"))
 (segment (start 14.4581 8.3456) (end 13.79 7.6775) (width 0.127) (layer "F.Cu") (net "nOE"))
 (segment (start 15.0277 8.3456) (end 14.4581 8.3456) (width 0.127) (layer "F.Cu") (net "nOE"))
 (via (at 15.0277 8.3456) (size 0.45) (drill 0.2) (layers "F.Cu" "B.Cu") (capping no) (covering (front no) (back no))
  (plugging (front no) (back no)) (filling no) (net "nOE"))
 (segment (start 4.795 23.845) (end 15.0277 13.6123) (width 0.127) (layer "B.Cu") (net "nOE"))
 (segment (start 15.0277 13.6123) (end 15.0277 8.3456) (width 0.127) (layer "B.Cu") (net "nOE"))
 (segment (start 13.1058 8.3125) (end 13.155 8.3125) (width 0.127) (layer "F.Cu") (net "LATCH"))
 (segment (start 13.155 8.3125) (end 13.79 8.9475) (width 0.127) (layer "F.Cu") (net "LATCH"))
 (via (at 13.1058 8.3125) (size 0.45) (drill 0.2) (layers "F.Cu" "B.Cu") (capping no) (covering (front no) (back no))
  (plugging (front no) (back no)) (filling no) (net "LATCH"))
 (segment (start 13.1058 12.9942) (end 4.795 21.305) (width 0.127) (layer "B.Cu") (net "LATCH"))
 (segment (start 13.1058 8.3125) (end 13.1058 12.9942) (width 0.127) (layer "B.Cu") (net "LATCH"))
 (segment (start 13.79 10.2175) (end 13.2095 10.2175) (width 0.127) (layer "F.Cu") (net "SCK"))
 (segment (start 13.2095 10.2175) (end 12.6611 10.7659) (width 0.127) (layer "F.Cu") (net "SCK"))
 (via (at 12.6611 10.7659) (size 0.45) (drill 0.2) (layers "F.Cu" "B.Cu") (capping no) (covering (front no) (back no))
  (plugging (front no) (back no)) (filling no) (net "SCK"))
 (segment (start 4.795 18.765) (end 12.6611 10.8989) (width 0.127) (layer "B.Cu") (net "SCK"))
 (segment (start 12.6611 10.8989) (end 12.6611 10.7659) (width 0.127) (layer "B.Cu") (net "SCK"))
 (segment (start 13.341 6.8565) (end 12.4634 6.8565) (width 0.127) (layer "F.Cu") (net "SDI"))
 (segment (start 13.79 6.4075) (end 13.341 6.8565) (width 0.127) (layer "F.Cu") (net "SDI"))
 (via (at 12.4634 6.8565) (size 0.45) (drill 0.2) (layers "F.Cu" "B.Cu") (capping no) (covering (front no) (back no))
  (plugging (front no) (back no)) (filling no) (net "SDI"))
 (segment (start 4.795 16.225) (end 5.0622 16.225) (width 0.127) (layer "B.Cu") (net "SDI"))
 (segment (start 5.0622 16.225) (end 12.4634 8.8238) (width 0.127) (layer "B.Cu") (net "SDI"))
 (segment (start 12.4634 8.8238) (end 12.4634 6.8565) (width 0.127) (layer "B.Cu") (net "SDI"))
 (segment (start 32.7537 3.1088) (end 35.4313 3.1088) (width 0.127) (layer "F.Cu") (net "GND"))
 (segment (start 19.5237 3.1088) (end 18.6575 3.975) (width 0.127) (layer "F.Cu") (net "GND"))
 (segment (start 49.5275 3.975) (end 48.6613 3.1088) (width 0.127) (layer "F.Cu") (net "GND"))
 (segment (start 6.8993 8.4286) (end 6.9769 8.5062) (width 0.127) (layer "F.Cu") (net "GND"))
 (segment (start 45.1175 3.975) (end 44.0211 2.8786) (width 0.127) (layer "F.Cu") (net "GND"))
 (segment (start 41.8039 2.8786) (end 40.7075 3.975) (width 0.127) (layer "F.Cu") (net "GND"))
 (segment (start 11.95 15.8675) (end 8.84 12.7575) (width 0.127) (layer "F.Cu") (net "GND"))
 (segment (start 15.0207 2.6093) (end 14.9714 2.56) (width 0.127) (layer "F.Cu") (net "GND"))
 (segment (start 14.0595 2.4357) (end 7.5043 2.4357) (width 0.127) (layer "F.Cu") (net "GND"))
 (segment (start 36.2975 3.975) (end 37.1637 3.1088) (width 0.127) (layer "F.Cu") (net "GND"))
 (segment (start 11.95 16) (end 11.95 15.8675) (width 0.127) (layer "F.Cu") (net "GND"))
 (segment (start 7.5043 2.4357) (end 6.7785 3.1615) (width 0.127) (layer "F.Cu") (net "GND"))
 (segment (start 23.0675 3.975) (end 22.2013 3.1088) (width 0.127) (layer "F.Cu") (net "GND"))
 (segment (start 22.2013 3.1088) (end 19.5237 3.1088) (width 0.127) (layer "F.Cu") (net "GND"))
 (segment (start 23.0675 3.975) (end 23.9337 3.1088) (width 0.127) (layer "F.Cu") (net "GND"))
 (segment (start 17.2918 2.6093) (end 15.0207 2.6093) (width 0.127) (layer "F.Cu") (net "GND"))
 (segment (start 28.3437 3.1088) (end 31.0213 3.1088) (width 0.127) (layer "F.Cu") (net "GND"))
 (segment (start 27.4775 3.975) (end 28.3437 3.1088) (width 0.127) (layer "F.Cu") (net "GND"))
 (segment (start 31.0213 3.1088) (end 31.8875 3.975) (width 0.127) (layer "F.Cu") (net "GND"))
 (segment (start 6.8993 8.3831) (end 6.8993 8.4286) (width 0.127) (layer "F.Cu") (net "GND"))
 (segment (start 14.9714 2.56) (end 14.1838 2.56) (width 0.127) (layer "F.Cu") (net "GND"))
 (segment (start 7.0075 11.4725) (end 4.795 13.685) (width 0.127) (layer "F.Cu") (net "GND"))
 (segment (start 26.6113 3.1088) (end 27.4775 3.975) (width 0.127) (layer "F.Cu") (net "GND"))
 (segment (start 35.4313 3.1088) (end 36.2975 3.975) (width 0.127) (layer "F.Cu") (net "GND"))
 (segment (start 14.1838 2.56) (end 14.0595 2.4357) (width 0.127) (layer "F.Cu") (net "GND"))
 (segment (start 6.7785 3.1615) (end 6.7785 8.2623) (width 0.127) (layer "F.Cu") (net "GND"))
 (segment (start 45.9837 3.1088) (end 45.1175 3.975) (width 0.127) (layer "F.Cu") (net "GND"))
 (segment (start 18.6575 3.975) (end 17.2918 2.6093) (width 0.127) (layer "F.Cu") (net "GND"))
 (segment (start 8.2924 12.7575) (end 7.0075 11.4725) (width 0.127) (layer "F.Cu") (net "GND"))
 (segment (start 44.0211 2.8786) (end 41.8039 2.8786) (width 0.127) (layer "F.Cu") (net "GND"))
 (segment (start 31.8875 3.975) (end 32.7537 3.1088) (width 0.127) (layer "F.Cu") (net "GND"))
 (segment (start 37.1637 3.1088) (end 39.8413 3.1088) (width 0.127) (layer "F.Cu") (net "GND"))
 (segment (start 23.9337 3.1088) (end 26.6113 3.1088) (width 0.127) (layer "F.Cu") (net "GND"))
 (segment (start 48.6613 3.1088) (end 45.9837 3.1088) (width 0.127) (layer "F.Cu") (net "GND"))
 (segment (start 8.84 12.7575) (end 8.2924 12.7575) (width 0.127) (layer "F.Cu") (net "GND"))
 (segment (start 6.9769 8.5062) (end 6.9769 11.442) (width 0.127) (layer "F.Cu") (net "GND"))
 (segment (start 39.8413 3.1088) (end 40.7075 3.975) (width 0.127) (layer "F.Cu") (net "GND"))
 (segment (start 6.9769 11.442) (end 7.0075 11.4725) (width 0.127) (layer "F.Cu") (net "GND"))
 (segment (start 6.7785 8.2623) (end 6.8993 8.3831) (width 0.127) (layer "F.Cu") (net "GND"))
 (segment (start 11.2016 9.5338) (end 11.2016 8.5952) (width 0.127) (layer "F.Cu") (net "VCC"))
 (segment (start 4.795 11.145) (end 4.795 12.1602) (width 0.127) (layer "F.Cu") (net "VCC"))
 (segment (start 8.879 14.829) (end 4.4831 14.829) (width 0.127) (layer "F.Cu") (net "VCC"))
 (segment (start 3.7798 14.1257) (end 3.7798 13.1754) (width 0.127) (layer "F.Cu") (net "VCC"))
 (segment (start 8.0468 7.1229) (end 7.6989 6.775) (width 0.127) (layer "F.Cu") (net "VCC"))
 (segment (start 10.05 16) (end 8.879 14.829) (width 0.127) (layer "F.Cu") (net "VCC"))
 (segment (start 12.8017 11.4875) (end 11.2016 9.8874) (width 0.127) (layer "F.Cu") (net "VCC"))
 (segment (start 11.2016 8.5952) (end 9.7293 7.1229) (width 0.127) (layer "F.Cu") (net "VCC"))
 (segment (start 7.6989 6.775) (end 7.6989 3.5565) (width 0.127) (layer "F.Cu") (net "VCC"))
 (segment (start 13.2906 3.3681) (end 13.79 3.8675) (width 0.127) (layer "F.Cu") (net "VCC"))
 (segment (start 9.7293 7.1229) (end 8.0468 7.1229) (width 0.127) (layer "F.Cu") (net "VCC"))
 (segment (start 7.6989 3.5565) (end 7.8873 3.3681) (width 0.127) (layer "F.Cu") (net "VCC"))
 (segment (start 13.79 11.4875) (end 12.8017 11.4875) (width 0.127) (layer "F.Cu") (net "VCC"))
 (segment (start 11.2016 9.8874) (end 11.2016 9.5338) (width 0.127) (layer "F.Cu") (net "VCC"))
 (segment (start 3.7798 13.1754) (end 4.795 12.1602) (width 0.127) (layer "F.Cu") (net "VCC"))
 (segment (start 4.4831 14.829) (end 3.7798 14.1257) (width 0.127) (layer "F.Cu") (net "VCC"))
 (segment (start 7.8873 3.3681) (end 13.2906 3.3681) (width 0.127) (layer "F.Cu") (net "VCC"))
 (via (at 11.2016 9.5338) (size 0.45) (drill 0.2) (layers "F.Cu" "B.Cu") (capping no) (covering (front no) (back no))
  (plugging (front no) (back no)) (filling no) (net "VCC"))
 (segment (start 7.4214 9.5338) (end 11.2016 9.5338) (width 0.127) (layer "B.Cu") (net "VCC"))
 (segment (start 4.795 11.145) (end 5.8102 11.145) (width 0.127) (layer "B.Cu") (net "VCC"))
 (segment (start 5.8102 11.145) (end 7.4214 9.5338) (width 0.127) (layer "B.Cu") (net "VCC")))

